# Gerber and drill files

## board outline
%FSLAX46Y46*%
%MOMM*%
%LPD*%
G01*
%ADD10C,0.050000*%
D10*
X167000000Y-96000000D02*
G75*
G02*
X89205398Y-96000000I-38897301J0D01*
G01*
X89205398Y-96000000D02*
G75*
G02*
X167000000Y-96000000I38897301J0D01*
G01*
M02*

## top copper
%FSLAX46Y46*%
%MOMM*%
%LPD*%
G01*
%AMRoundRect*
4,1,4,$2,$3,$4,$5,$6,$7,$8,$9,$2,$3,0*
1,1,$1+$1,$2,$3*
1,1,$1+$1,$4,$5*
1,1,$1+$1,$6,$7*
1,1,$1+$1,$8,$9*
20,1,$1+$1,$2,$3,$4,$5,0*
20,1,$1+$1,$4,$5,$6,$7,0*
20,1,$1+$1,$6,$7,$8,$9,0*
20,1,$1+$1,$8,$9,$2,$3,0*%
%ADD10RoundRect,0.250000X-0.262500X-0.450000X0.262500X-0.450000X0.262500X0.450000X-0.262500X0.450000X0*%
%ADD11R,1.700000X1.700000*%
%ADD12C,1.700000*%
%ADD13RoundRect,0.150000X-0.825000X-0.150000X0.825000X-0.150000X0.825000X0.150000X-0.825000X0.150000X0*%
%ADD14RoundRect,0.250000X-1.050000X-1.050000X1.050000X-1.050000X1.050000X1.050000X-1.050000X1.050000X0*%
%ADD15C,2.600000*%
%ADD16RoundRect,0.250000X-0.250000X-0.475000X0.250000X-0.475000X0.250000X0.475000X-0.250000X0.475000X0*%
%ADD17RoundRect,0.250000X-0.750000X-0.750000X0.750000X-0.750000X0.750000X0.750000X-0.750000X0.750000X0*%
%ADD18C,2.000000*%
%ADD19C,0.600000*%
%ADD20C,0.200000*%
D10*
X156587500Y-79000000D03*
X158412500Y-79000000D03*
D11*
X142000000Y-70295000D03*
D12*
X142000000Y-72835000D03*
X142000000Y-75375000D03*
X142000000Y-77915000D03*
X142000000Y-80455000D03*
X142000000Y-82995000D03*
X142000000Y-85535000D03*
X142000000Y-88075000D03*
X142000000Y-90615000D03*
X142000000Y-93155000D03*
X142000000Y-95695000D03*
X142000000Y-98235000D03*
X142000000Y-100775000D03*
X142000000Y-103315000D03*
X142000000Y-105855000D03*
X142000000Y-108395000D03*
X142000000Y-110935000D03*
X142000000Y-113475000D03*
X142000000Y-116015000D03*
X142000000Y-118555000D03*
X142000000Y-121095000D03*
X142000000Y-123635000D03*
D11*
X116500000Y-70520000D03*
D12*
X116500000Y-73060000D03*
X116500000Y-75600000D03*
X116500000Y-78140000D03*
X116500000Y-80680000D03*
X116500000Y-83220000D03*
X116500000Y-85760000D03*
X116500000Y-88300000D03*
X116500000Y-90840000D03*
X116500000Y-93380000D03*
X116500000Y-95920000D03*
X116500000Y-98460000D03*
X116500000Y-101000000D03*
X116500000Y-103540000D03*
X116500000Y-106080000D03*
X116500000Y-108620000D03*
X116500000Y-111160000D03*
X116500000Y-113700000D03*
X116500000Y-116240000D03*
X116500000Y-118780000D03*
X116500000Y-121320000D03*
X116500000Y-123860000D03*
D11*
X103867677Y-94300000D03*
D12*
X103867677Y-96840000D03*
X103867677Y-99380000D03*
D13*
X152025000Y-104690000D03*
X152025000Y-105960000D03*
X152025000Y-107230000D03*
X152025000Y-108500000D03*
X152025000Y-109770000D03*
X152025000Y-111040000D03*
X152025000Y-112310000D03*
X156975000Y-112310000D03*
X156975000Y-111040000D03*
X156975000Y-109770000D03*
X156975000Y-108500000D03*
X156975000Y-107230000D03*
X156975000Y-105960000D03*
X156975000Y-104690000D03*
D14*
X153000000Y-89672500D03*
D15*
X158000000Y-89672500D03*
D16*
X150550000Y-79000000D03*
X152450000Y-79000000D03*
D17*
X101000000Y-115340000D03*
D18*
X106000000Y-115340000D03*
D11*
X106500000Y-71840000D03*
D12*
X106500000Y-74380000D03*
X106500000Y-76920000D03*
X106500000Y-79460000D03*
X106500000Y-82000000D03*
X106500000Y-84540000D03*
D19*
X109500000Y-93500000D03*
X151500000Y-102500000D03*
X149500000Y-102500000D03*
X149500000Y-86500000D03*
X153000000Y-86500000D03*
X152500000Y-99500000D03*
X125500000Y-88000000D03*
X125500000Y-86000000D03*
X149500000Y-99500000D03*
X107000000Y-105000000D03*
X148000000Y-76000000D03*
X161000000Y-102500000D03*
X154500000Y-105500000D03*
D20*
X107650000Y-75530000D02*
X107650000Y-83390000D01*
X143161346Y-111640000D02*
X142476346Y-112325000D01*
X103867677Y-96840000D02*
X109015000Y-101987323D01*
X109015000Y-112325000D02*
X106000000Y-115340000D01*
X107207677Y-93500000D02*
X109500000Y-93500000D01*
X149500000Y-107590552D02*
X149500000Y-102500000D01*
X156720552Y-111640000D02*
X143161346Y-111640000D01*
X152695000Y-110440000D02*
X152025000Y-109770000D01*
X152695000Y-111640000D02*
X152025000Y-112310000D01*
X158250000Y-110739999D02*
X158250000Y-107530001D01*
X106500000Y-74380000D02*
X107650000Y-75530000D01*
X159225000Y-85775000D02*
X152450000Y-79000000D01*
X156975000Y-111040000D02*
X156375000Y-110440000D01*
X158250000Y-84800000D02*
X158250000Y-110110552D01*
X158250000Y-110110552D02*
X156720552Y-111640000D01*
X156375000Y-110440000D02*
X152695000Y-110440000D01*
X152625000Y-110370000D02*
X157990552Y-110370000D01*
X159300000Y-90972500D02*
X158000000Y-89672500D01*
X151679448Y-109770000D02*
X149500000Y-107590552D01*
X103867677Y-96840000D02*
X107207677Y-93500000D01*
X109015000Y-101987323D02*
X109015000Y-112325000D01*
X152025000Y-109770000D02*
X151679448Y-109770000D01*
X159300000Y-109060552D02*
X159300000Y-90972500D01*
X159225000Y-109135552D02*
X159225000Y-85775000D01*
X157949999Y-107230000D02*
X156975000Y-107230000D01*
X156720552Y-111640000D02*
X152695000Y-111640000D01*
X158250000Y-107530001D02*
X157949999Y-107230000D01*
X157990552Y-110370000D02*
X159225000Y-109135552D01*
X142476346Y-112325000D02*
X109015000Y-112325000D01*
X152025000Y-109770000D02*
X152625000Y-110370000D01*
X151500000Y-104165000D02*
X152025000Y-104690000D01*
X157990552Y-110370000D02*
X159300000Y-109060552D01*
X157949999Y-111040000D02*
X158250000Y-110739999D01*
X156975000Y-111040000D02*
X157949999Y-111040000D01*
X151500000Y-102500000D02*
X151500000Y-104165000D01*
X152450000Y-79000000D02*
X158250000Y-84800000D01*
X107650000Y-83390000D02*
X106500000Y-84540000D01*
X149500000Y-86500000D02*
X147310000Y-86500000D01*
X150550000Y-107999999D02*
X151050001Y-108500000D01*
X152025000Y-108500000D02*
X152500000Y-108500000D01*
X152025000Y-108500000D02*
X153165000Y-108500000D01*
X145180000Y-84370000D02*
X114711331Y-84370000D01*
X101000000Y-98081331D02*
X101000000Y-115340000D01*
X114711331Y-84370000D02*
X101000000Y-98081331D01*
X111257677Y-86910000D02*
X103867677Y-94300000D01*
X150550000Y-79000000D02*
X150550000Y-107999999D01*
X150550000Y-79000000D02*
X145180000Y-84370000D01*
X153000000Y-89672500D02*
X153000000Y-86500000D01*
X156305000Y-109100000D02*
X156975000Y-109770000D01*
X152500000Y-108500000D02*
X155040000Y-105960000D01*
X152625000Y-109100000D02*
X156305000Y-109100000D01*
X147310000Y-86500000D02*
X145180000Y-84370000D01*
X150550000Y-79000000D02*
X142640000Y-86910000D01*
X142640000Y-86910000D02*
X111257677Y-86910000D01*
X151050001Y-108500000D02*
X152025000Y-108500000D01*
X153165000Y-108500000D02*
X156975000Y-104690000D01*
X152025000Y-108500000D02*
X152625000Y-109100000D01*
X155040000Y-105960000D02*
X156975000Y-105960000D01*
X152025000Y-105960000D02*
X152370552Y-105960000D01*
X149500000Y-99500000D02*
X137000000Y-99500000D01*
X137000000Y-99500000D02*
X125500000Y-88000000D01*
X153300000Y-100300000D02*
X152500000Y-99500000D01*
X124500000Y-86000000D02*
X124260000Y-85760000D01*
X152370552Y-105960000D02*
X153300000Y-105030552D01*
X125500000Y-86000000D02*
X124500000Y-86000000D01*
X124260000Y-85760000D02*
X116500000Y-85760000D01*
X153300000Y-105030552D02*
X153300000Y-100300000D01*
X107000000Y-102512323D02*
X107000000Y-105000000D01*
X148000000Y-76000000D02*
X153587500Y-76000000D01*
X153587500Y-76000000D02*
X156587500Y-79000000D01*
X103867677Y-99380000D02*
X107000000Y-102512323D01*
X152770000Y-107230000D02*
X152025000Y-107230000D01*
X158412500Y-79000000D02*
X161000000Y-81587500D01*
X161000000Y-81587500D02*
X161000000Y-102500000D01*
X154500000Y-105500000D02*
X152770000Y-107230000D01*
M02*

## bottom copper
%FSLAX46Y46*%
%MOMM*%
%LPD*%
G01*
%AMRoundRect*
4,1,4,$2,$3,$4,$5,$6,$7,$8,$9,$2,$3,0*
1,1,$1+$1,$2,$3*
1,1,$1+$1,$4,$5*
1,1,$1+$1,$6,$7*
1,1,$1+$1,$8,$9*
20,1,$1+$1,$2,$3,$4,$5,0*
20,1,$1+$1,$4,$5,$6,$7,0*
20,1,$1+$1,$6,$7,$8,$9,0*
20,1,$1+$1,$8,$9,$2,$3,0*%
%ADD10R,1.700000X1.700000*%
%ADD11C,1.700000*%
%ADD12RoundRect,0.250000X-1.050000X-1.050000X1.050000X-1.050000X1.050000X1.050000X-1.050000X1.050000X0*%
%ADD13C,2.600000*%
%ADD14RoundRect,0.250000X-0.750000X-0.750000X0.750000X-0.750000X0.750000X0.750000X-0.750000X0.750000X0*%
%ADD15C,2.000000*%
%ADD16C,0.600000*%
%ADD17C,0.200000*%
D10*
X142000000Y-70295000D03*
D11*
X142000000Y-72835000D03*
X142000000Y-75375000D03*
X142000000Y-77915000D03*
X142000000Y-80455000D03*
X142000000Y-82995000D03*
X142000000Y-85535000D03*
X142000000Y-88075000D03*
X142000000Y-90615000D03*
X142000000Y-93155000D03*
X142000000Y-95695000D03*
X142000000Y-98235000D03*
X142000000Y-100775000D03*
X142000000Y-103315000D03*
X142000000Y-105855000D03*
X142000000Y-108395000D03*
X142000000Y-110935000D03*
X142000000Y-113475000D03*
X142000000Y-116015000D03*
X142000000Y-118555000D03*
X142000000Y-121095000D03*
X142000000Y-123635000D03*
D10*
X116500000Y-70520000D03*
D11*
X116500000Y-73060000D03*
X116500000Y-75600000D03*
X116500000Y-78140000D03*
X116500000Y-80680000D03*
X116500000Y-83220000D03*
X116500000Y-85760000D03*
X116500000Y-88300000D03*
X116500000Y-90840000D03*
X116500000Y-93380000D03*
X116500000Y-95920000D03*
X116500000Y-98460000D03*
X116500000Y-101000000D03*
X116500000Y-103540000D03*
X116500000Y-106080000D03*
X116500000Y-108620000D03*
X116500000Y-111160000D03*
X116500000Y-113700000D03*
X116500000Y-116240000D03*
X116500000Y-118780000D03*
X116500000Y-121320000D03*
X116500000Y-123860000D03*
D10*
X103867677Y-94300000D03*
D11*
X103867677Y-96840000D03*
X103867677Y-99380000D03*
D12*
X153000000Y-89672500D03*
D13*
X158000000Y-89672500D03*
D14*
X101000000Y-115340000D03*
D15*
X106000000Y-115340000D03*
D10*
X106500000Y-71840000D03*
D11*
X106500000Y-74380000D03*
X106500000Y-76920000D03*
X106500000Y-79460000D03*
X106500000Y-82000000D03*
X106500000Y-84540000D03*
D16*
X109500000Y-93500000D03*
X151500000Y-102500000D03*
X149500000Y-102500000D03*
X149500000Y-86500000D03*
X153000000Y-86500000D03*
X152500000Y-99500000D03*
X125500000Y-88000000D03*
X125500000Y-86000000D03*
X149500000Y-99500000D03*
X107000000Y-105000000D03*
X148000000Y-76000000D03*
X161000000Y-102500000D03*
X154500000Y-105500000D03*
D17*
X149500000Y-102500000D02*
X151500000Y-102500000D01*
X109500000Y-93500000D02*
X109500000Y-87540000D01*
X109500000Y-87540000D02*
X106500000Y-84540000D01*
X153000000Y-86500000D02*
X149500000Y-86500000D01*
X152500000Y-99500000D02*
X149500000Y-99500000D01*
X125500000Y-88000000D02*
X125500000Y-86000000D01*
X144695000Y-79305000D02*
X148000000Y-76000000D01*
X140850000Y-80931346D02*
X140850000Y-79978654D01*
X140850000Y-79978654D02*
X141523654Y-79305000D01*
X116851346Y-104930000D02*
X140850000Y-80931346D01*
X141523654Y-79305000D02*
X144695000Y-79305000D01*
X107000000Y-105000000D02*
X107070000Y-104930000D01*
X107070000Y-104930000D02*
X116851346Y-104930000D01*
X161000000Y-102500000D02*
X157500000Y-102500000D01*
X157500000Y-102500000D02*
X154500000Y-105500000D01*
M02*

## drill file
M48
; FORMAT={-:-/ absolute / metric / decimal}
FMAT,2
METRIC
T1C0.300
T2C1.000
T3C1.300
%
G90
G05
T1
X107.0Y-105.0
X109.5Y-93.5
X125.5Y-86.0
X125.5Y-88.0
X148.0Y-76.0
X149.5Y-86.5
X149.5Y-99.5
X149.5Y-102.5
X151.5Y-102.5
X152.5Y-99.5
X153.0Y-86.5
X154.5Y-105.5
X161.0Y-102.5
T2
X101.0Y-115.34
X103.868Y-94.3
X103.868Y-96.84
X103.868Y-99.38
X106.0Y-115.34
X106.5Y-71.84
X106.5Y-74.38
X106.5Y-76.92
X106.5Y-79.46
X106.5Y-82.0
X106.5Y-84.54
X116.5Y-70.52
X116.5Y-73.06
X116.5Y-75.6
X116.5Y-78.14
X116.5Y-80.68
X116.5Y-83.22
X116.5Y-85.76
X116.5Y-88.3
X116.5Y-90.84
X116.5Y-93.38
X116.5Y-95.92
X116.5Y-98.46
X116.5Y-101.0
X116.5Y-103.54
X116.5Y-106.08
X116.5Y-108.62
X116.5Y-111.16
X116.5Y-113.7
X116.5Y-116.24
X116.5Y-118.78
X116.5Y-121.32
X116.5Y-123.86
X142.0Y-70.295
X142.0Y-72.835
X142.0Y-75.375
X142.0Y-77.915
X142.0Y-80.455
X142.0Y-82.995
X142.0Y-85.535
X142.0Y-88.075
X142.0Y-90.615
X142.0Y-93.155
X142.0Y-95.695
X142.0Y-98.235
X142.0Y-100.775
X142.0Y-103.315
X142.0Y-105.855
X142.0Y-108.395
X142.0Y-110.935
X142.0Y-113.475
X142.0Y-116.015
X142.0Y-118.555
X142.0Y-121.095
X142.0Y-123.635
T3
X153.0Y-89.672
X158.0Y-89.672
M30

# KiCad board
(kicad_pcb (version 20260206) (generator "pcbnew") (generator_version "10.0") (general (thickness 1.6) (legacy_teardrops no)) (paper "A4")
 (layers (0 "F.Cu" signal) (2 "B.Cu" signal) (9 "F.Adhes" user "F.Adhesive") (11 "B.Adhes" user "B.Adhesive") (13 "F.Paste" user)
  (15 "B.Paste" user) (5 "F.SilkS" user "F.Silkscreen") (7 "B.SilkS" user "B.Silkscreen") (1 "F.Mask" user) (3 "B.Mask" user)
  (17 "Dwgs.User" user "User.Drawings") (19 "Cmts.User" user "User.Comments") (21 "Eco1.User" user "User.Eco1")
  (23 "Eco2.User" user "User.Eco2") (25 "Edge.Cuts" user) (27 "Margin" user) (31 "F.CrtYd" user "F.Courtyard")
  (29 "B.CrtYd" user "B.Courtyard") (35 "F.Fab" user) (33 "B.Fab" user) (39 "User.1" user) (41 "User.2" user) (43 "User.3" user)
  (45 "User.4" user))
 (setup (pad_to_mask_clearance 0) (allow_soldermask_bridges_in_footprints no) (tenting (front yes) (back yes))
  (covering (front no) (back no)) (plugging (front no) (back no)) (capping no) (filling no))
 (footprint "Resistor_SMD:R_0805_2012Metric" (layer "F.Cu") (at 157.5 79)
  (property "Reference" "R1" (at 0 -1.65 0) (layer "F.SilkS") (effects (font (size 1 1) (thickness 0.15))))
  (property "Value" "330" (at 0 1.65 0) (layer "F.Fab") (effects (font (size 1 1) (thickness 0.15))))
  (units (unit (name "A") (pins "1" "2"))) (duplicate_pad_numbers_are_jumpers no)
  (pad "1" smd roundrect (at -0.9125 0) (size 1.025 1.4) (layers "F.Cu" "F.Mask" "F.Paste") (roundrect_rratio 0.243902)
   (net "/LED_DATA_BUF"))
  (pad "2" smd roundrect (at 0.9125 0) (size 1.025 1.4) (layers "F.Cu" "F.Mask" "F.Paste") (roundrect_rratio 0.243902) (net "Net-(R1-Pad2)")))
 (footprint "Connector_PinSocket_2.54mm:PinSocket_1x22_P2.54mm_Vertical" (layer "F.Cu") (at 142 70.295)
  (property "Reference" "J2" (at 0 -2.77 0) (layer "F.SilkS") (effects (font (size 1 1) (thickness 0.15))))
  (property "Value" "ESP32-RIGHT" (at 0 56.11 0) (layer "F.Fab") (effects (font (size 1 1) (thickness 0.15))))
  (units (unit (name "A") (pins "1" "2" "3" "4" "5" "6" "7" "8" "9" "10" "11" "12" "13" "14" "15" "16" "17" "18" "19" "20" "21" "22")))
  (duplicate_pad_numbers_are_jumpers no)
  (pad "1" thru_hole rect (at 0 0) (size 1.7 1.7) (drill 1) (layers "*.Cu" "*.Mask") (remove_unused_layers no)
   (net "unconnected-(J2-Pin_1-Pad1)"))
  (pad "2" thru_hole circle (at 0 2.54) (size 1.7 1.7) (drill 1) (layers "*.Cu" "*.Mask") (remove_unused_layers no)
   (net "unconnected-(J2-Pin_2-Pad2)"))
  (pad "3" thru_hole circle (at 0 5.08) (size 1.7 1.7) (drill 1) (layers "*.Cu" "*.Mask") (remove_unused_layers no)
   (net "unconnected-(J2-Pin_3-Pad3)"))
  (pad "4" thru_hole circle (at 0 7.62) (size 1.7 1.7) (drill 1) (layers "*.Cu" "*.Mask") (remove_unused_layers no)
   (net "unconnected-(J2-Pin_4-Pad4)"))
  (pad "5" thru_hole circle (at 0 10.16) (size 1.7 1.7) (drill 1) (layers "*.Cu" "*.Mask") (remove_unused_layers no)
   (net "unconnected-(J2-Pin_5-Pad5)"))
  (pad "6" thru_hole circle (at 0 12.7) (size 1.7 1.7) (drill 1) (layers "*.Cu" "*.Mask") (remove_unused_layers no)
   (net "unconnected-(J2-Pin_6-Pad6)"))
  (pad "7" thru_hole circle (at 0 15.24) (size 1.7 1.7) (drill 1) (layers "*.Cu" "*.Mask") (remove_unused_layers no)
   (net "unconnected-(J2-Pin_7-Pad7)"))
  (pad "8" thru_hole circle (at 0 17.78) (size 1.7 1.7) (drill 1) (layers "*.Cu" "*.Mask") (remove_unused_layers no)
   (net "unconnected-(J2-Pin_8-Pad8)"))
  (pad "9" thru_hole circle (at 0 20.32) (size 1.7 1.7) (drill 1) (layers "*.Cu" "*.Mask") (remove_unused_layers no)
   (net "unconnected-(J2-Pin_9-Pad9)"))
  (pad "10" thru_hole circle (at 0 22.86) (size 1.7 1.7) (drill 1) (layers "*.Cu" "*.Mask") (remove_unused_layers no)
   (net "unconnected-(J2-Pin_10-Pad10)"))
  (pad "11" thru_hole circle (at 0 25.4) (size 1.7 1.7) (drill 1) (layers "*.Cu" "*.Mask") (remove_unused_layers no)
   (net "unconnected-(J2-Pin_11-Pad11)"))
  (pad "12" thru_hole circle (at 0 27.94) (size 1.7 1.7) (drill 1) (layers "*.Cu" "*.Mask") (remove_unused_layers no)
   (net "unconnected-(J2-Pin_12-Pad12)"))
  (pad "13" thru_hole circle (at 0 30.48) (size 1.7 1.7) (drill 1) (layers "*.Cu" "*.Mask") (remove_unused_layers no)
   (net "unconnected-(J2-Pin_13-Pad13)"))
  (pad "14" thru_hole circle (at 0 33.02) (size 1.7 1.7) (drill 1) (layers "*.Cu" "*.Mask") (remove_unused_layers no)
   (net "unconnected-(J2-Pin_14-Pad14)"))
  (pad "15" thru_hole circle (at 0 35.56) (size 1.7 1.7) (drill 1) (layers "*.Cu" "*.Mask") (remove_unused_layers no)
   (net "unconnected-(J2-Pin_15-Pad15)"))
  (pad "16" thru_hole circle (at 0 38.1) (size 1.7 1.7) (drill 1) (layers "*.Cu" "*.Mask") (remove_unused_layers no)
   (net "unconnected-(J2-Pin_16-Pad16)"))
  (pad "17" thru_hole circle (at 0 40.64) (size 1.7 1.7) (drill 1) (layers "*.Cu" "*.Mask") (remove_unused_layers no)
   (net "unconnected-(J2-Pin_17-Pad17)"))
  (pad "18" thru_hole circle (at 0 43.18) (size 1.7 1.7) (drill 1) (layers "*.Cu" "*.Mask") (remove_unused_layers no)
   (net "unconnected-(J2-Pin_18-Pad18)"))
  (pad "19" thru_hole circle (at 0 45.72) (size 1.7 1.7) (drill 1) (layers "*.Cu" "*.Mask") (remove_unused_layers no)
   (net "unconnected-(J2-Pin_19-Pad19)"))
  (pad "20" thru_hole circle (at 0 48.26) (size 1.7 1.7) (drill 1) (layers "*.Cu" "*.Mask") (remove_unused_layers no)
   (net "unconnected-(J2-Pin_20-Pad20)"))
  (pad "21" thru_hole circle (at 0 50.8) (size 1.7 1.7) (drill 1) (layers "*.Cu" "*.Mask") (remove_unused_layers no)
   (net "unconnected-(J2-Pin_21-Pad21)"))
  (pad "22" thru_hole circle (at 0 53.34) (size 1.7 1.7) (drill 1) (layers "*.Cu" "*.Mask") (remove_unused_layers no)
   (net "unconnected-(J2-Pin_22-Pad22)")))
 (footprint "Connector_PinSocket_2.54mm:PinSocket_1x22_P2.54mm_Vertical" (layer "F.Cu") (at 116.5 70.52)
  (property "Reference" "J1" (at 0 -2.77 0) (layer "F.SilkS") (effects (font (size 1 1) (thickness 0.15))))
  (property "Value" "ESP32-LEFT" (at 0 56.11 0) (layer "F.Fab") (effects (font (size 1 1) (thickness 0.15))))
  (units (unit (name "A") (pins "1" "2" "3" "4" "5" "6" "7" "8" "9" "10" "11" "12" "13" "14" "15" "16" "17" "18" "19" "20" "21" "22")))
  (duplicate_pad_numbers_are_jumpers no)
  (pad "1" thru_hole rect (at 0 0) (size 1.7 1.7) (drill 1) (layers "*.Cu" "*.Mask") (remove_unused_layers no)
   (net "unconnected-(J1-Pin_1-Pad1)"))
  (pad "2" thru_hole circle (at 0 2.54) (size 1.7 1.7) (drill 1) (layers "*.Cu" "*.Mask") (remove_unused_layers no)
   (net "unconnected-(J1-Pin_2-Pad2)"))
  (pad "3" thru_hole circle (at 0 5.08) (size 1.7 1.7) (drill 1) (layers "*.Cu" "*.Mask") (remove_unused_layers no)
   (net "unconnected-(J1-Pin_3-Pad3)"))
  (pad "4" thru_hole circle (at 0 7.62) (size 1.7 1.7) (drill 1) (layers "*.Cu" "*.Mask") (remove_unused_layers no)
   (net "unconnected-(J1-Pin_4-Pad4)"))
  (pad "5" thru_hole circle (at 0 10.16) (size 1.7 1.7) (drill 1) (layers "*.Cu" "*.Mask") (remove_unused_layers no)
   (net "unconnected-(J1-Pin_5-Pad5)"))
  (pad "6" thru_hole circle (at 0 12.7) (size 1.7 1.7) (drill 1) (layers "*.Cu" "*.Mask") (remove_unused_layers no)
   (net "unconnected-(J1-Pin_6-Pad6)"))
  (pad "7" thru_hole circle (at 0 15.24) (size 1.7 1.7) (drill 1) (layers "*.Cu" "*.Mask") (remove_unused_layers no) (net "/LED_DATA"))
  (pad "8" thru_hole circle (at 0 17.78) (size 1.7 1.7) (drill 1) (layers "*.Cu" "*.Mask") (remove_unused_layers no)
   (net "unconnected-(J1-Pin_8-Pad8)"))
  (pad "9" thru_hole circle (at 0 20.32) (size 1.7 1.7) (drill 1) (layers "*.Cu" "*.Mask") (remove_unused_layers no)
   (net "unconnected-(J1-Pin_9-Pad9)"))
  (pad "10" thru_hole circle (at 0 22.86) (size 1.7 1.7) (drill 1) (layers "*.Cu" "*.Mask") (remove_unused_layers no)
   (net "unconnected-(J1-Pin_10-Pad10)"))
  (pad "11" thru_hole circle (at 0 25.4) (size 1.7 1.7) (drill 1) (layers "*.Cu" "*.Mask") (remove_unused_layers no)
   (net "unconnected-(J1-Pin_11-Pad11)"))
  (pad "12" thru_hole circle (at 0 27.94) (size 1.7 1.7) (drill 1) (layers "*.Cu" "*.Mask") (remove_unused_layers no)
   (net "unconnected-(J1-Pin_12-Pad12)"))
  (pad "13" thru_hole circle (at 0 30.48) (size 1.7 1.7) (drill 1) (layers "*.Cu" "*.Mask") (remove_unused_layers no)
   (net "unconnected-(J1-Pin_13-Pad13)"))
  (pad "14" thru_hole circle (at 0 33.02) (size 1.7 1.7) (drill 1) (layers "*.Cu" "*.Mask") (remove_unused_layers no)
   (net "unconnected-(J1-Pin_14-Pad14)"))
  (pad "15" thru_hole circle (at 0 35.56) (size 1.7 1.7) (drill 1) (layers "*.Cu" "*.Mask") (remove_unused_layers no)
   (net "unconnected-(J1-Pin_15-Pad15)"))
  (pad "16" thru_hole circle (at 0 38.1) (size 1.7 1.7) (drill 1) (layers "*.Cu" "*.Mask") (remove_unused_layers no)
   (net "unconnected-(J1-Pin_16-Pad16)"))
  (pad "17" thru_hole circle (at 0 40.64) (size 1.7 1.7) (drill 1) (layers "*.Cu" "*.Mask") (remove_unused_layers no)
   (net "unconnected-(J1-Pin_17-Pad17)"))
  (pad "18" thru_hole circle (at 0 43.18) (size 1.7 1.7) (drill 1) (layers "*.Cu" "*.Mask") (remove_unused_layers no)
   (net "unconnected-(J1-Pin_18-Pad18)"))
  (pad "19" thru_hole circle (at 0 45.72) (size 1.7 1.7) (drill 1) (layers "*.Cu" "*.Mask") (remove_unused_layers no)
   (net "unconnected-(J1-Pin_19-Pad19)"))
  (pad "20" thru_hole circle (at 0 48.26) (size 1.7 1.7) (drill 1) (layers "*.Cu" "*.Mask") (remove_unused_layers no)
   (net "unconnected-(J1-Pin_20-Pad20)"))
  (pad "21" thru_hole circle (at 0 50.8) (size 1.7 1.7) (drill 1) (layers "*.Cu" "*.Mask") (remove_unused_layers no)
   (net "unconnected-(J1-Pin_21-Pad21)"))
  (pad "22" thru_hole circle (at 0 53.34) (size 1.7 1.7) (drill 1) (layers "*.Cu" "*.Mask") (remove_unused_layers no)
   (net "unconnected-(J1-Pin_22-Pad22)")))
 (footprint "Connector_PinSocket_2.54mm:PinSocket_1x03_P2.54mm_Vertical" (layer "F.Cu") (at 103.867677 94.3)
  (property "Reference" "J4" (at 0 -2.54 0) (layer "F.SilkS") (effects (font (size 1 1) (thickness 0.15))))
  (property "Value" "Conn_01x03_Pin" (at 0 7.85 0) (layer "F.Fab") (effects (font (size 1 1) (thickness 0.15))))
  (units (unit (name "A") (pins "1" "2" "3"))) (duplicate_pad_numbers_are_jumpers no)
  (pad "1" thru_hole rect (at 0 0) (size 1.7 1.7) (drill 1) (layers "*.Cu" "*.Mask") (remove_unused_layers no) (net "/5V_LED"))
  (pad "2" thru_hole circle (at 0 2.54) (size 1.7 1.7) (drill 1) (layers "*.Cu" "*.Mask") (remove_unused_layers no) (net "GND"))
  (pad "3" thru_hole circle (at 0 5.08) (size 1.7 1.7) (drill 1) (layers "*.Cu" "*.Mask") (remove_unused_layers no) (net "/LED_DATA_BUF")))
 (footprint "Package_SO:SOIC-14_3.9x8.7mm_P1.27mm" (layer "F.Cu") (at 154.5 108.5)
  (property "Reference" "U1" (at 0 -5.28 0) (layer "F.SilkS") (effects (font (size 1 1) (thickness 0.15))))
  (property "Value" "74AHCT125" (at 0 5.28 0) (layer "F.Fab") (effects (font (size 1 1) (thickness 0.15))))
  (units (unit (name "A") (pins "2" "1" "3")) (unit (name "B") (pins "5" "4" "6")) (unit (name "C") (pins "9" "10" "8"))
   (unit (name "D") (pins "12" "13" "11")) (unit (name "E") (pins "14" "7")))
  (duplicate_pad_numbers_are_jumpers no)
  (pad "1" smd roundrect (at -2.475 -3.81) (size 1.95 0.6) (layers "F.Cu" "F.Mask" "F.Paste") (roundrect_rratio 0.25) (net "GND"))
  (pad "2" smd roundrect (at -2.475 -2.54) (size 1.95 0.6) (layers "F.Cu" "F.Mask" "F.Paste") (roundrect_rratio 0.25) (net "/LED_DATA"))
  (pad "3" smd roundrect (at -2.475 -1.27) (size 1.95 0.6) (layers "F.Cu" "F.Mask" "F.Paste") (roundrect_rratio 0.25) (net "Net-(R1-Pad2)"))
  (pad "4" smd roundrect (at -2.475 0) (size 1.95 0.6) (layers "F.Cu" "F.Mask" "F.Paste") (roundrect_rratio 0.25) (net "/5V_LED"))
  (pad "5" smd roundrect (at -2.475 1.27) (size 1.95 0.6) (layers "F.Cu" "F.Mask" "F.Paste") (roundrect_rratio 0.25) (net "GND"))
  (pad "6" smd roundrect (at -2.475 2.54) (size 1.95 0.6) (layers "F.Cu" "F.Mask" "F.Paste") (roundrect_rratio 0.25)
   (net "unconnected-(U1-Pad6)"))
  (pad "7" smd roundrect (at -2.475 3.81) (size 1.95 0.6) (layers "F.Cu" "F.Mask" "F.Paste") (roundrect_rratio 0.25) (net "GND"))
  (pad "8" smd roundrect (at 2.475 3.81) (size 1.95 0.6) (layers "F.Cu" "F.Mask" "F.Paste") (roundrect_rratio 0.25)
   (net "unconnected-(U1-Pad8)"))
  (pad "9" smd roundrect (at 2.475 2.54) (size 1.95 0.6) (layers "F.Cu" "F.Mask" "F.Paste") (roundrect_rratio 0.25) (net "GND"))
  (pad "10" smd roundrect (at 2.475 1.27) (size 1.95 0.6) (layers "F.Cu" "F.Mask" "F.Paste") (roundrect_rratio 0.25) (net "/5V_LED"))
  (pad "11" smd roundrect (at 2.475 0) (size 1.95 0.6) (layers "F.Cu" "F.Mask" "F.Paste") (roundrect_rratio 0.25)
   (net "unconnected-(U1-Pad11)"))
  (pad "12" smd roundrect (at 2.475 -1.27) (size 1.95 0.6) (layers "F.Cu" "F.Mask" "F.Paste") (roundrect_rratio 0.25) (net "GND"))
  (pad "13" smd roundrect (at 2.475 -2.54) (size 1.95 0.6) (layers "F.Cu" "F.Mask" "F.Paste") (roundrect_rratio 0.25) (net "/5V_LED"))
  (pad "14" smd roundrect (at 2.475 -3.81) (size 1.95 0.6) (layers "F.Cu" "F.Mask" "F.Paste") (roundrect_rratio 0.25) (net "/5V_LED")))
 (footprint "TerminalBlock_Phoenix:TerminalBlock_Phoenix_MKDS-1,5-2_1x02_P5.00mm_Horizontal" (layer "F.Cu") (at 153 89.6725)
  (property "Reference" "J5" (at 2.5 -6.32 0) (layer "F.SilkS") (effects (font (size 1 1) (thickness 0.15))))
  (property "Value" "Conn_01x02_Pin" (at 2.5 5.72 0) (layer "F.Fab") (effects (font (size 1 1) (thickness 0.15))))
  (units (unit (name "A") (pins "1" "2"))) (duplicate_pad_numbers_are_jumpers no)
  (pad "1" thru_hole roundrect (at 0 0) (size 2.6 2.6) (drill 1.3) (layers "*.Cu" "*.Mask") (remove_unused_layers no)
   (roundrect_rratio 0.096154) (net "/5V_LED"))
  (pad "2" thru_hole circle (at 5 0) (size 2.6 2.6) (drill 1.3) (layers "*.Cu" "*.Mask") (remove_unused_layers no) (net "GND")))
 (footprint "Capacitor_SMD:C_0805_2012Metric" (layer "F.Cu") (at 151.5 79)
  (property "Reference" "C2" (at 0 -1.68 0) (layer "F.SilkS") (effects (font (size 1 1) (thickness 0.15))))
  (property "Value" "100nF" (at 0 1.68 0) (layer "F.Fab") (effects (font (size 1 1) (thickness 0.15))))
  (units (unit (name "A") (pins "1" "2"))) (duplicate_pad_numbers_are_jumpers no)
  (pad "1" smd roundrect (at -0.95 0) (size 1 1.45) (layers "F.Cu" "F.Mask" "F.Paste") (roundrect_rratio 0.25) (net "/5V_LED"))
  (pad "2" smd roundrect (at 0.95 0) (size 1 1.45) (layers "F.Cu" "F.Mask" "F.Paste") (roundrect_rratio 0.25) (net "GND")))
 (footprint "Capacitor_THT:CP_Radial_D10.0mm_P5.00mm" (layer "F.Cu") (at 101 115.34)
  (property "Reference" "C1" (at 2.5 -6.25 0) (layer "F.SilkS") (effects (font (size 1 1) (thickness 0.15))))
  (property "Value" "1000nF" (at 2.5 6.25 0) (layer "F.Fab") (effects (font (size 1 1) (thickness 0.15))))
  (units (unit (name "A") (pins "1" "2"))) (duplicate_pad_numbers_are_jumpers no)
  (pad "1" thru_hole roundrect (at 0 0) (size 2 2) (drill 1) (layers "*.Cu" "*.Mask") (remove_unused_layers no) (roundrect_rratio 0.125)
   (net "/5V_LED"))
  (pad "2" thru_hole circle (at 5 0) (size 2 2) (drill 1) (layers "*.Cu" "*.Mask") (remove_unused_layers no) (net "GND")))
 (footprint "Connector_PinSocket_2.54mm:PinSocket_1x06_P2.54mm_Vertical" (layer "F.Cu") (at 106.5 71.84)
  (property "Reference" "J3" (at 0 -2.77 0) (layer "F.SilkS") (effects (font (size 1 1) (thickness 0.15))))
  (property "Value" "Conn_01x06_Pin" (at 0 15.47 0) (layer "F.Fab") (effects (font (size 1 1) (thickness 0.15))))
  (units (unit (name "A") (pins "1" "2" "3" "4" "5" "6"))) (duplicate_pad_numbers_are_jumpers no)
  (pad "1" thru_hole rect (at 0 0) (size 1.7 1.7) (drill 1) (layers "*.Cu" "*.Mask") (remove_unused_layers no) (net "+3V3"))
  (pad "2" thru_hole circle (at 0 2.54) (size 1.7 1.7) (drill 1) (layers "*.Cu" "*.Mask") (remove_unused_layers no) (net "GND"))
  (pad "3" thru_hole circle (at 0 5.08) (size 1.7 1.7) (drill 1) (layers "*.Cu" "*.Mask") (remove_unused_layers no) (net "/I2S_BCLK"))
  (pad "4" thru_hole circle (at 0 7.62) (size 1.7 1.7) (drill 1) (layers "*.Cu" "*.Mask") (remove_unused_layers no) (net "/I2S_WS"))
  (pad "5" thru_hole circle (at 0 10.16) (size 1.7 1.7) (drill 1) (layers "*.Cu" "*.Mask") (remove_unused_layers no) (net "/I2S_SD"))
  (pad "6" thru_hole circle (at 0 12.7) (size 1.7 1.7) (drill 1) (layers "*.Cu" "*.Mask") (remove_unused_layers no) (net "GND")))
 (gr_circle (center 128.102699 96) (end 155.102699 124) (stroke (width 0.05) (type default)) (fill no) (layer "Edge.Cuts"))
 (segment (start 107.65 75.53) (end 107.65 83.39) (width 0.2) (layer "F.Cu") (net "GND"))
 (segment (start 143.161346 111.64) (end 142.476346 112.325) (width 0.2) (layer "F.Cu") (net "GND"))
 (segment (start 103.867677 96.84) (end 109.015 101.987323) (width 0.2) (layer "F.Cu") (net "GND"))
 (segment (start 109.015 112.325) (end 106 115.34) (width 0.2) (layer "F.Cu") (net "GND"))
 (segment (start 107.207677 93.5) (end 109.5 93.5) (width 0.2) (layer "F.Cu") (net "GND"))
 (segment (start 149.5 107.590552) (end 149.5 102.5) (width 0.2) (layer "F.Cu") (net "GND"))
 (segment (start 156.720552 111.64) (end 143.161346 111.64) (width 0.2) (layer "F.Cu") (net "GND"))
 (segment (start 152.695 110.44) (end 152.025 109.77) (width 0.2) (layer "F.Cu") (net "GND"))
 (segment (start 152.695 111.64) (end 152.025 112.31) (width 0.2) (layer "F.Cu") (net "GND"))
 (segment (start 158.25 110.739999) (end 158.25 107.530001) (width 0.2) (layer "F.Cu") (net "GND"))
 (segment (start 106.5 74.38) (end 107.65 75.53) (width 0.2) (layer "F.Cu") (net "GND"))
 (segment (start 159.225 85.775) (end 152.45 79) (width 0.2) (layer "F.Cu") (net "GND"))
 (segment (start 156.975 111.04) (end 156.375 110.44) (width 0.2) (layer "F.Cu") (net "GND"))
 (segment (start 158.25 84.8) (end 158.25 110.110552) (width 0.2) (layer "F.Cu") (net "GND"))
 (segment (start 158.25 110.110552) (end 156.720552 111.64) (width 0.2) (layer "F.Cu") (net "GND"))
 (segment (start 156.375 110.44) (end 152.695 110.44) (width 0.2) (layer "F.Cu") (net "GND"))
 (segment (start 152.625 110.37) (end 157.990552 110.37) (width 0.2) (layer "F.Cu") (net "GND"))
 (segment (start 159.3 90.9725) (end 158 89.6725) (width 0.2) (layer "F.Cu") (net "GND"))
 (segment (start 151.679448 109.77) (end 149.5 107.590552) (width 0.2) (layer "F.Cu") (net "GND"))
 (segment (start 103.867677 96.84) (end 107.207677 93.5) (width 0.2) (layer "F.Cu") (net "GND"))
 (segment (start 109.015 101.987323) (end 109.015 112.325) (width 0.2) (layer "F.Cu") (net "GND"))
 (segment (start 152.025 109.77) (end 151.679448 109.77) (width 0.2) (layer "F.Cu") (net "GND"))
 (segment (start 159.3 109.060552) (end 159.3 90.9725) (width 0.2) (layer "F.Cu") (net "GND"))
 (segment (start 159.225 109.135552) (end 159.225 85.775) (width 0.2) (layer "F.Cu") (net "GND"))
 (segment (start 157.949999 107.23) (end 156.975 107.23) (width 0.2) (layer "F.Cu") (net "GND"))
 (segment (start 156.720552 111.64) (end 152.695 111.64) (width 0.2) (layer "F.Cu") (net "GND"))
 (segment (start 158.25 107.530001) (end 157.949999 107.23) (width 0.2) (layer "F.Cu") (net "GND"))
 (segment (start 157.990552 110.37) (end 159.225 109.135552) (width 0.2) (layer "F.Cu") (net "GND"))
 (segment (start 142.476346 112.325) (end 109.015 112.325) (width 0.2) (layer "F.Cu") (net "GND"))
 (segment (start 152.025 109.77) (end 152.625 110.37) (width 0.2) (layer "F.Cu") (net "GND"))
 (segment (start 151.5 104.165) (end 152.025 104.69) (width 0.2) (layer "F.Cu") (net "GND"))
 (segment (start 157.990552 110.37) (end 159.3 109.060552) (width 0.2) (layer "F.Cu") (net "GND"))
 (segment (start 157.949999 111.04) (end 158.25 110.739999) (width 0.2) (layer "F.Cu") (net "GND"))
 (segment (start 156.975 111.04) (end 157.949999 111.04) (width 0.2) (layer "F.Cu") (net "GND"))
 (segment (start 151.5 102.5) (end 151.5 104.165) (width 0.2) (layer "F.Cu") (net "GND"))
 (segment (start 152.45 79) (end 158.25 84.8) (width 0.2) (layer "F.Cu") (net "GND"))
 (segment (start 107.65 83.39) (end 106.5 84.54) (width 0.2) (layer "F.Cu") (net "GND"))
 (via (at 109.5 93.5) (size 0.6) (drill 0.3) (layers "F.Cu" "B.Cu") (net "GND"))
 (via (at 151.5 102.5) (size 0.6) (drill 0.3) (layers "F.Cu" "B.Cu") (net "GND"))
 (via (at 149.5 102.5) (size 0.6) (drill 0.3) (layers "F.Cu" "B.Cu") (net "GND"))
 (segment (start 149.5 102.5) (end 151.5 102.5) (width 0.2) (layer "B.Cu") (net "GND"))
 (segment (start 109.5 93.5) (end 109.5 87.54) (width 0.2) (layer "B.Cu") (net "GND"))
 (segment (start 109.5 87.54) (end 106.5 84.54) (width 0.2) (layer "B.Cu") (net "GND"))
 (segment (start 149.5 86.5) (end 147.31 86.5) (width 0.2) (layer "F.Cu") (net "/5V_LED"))
 (segment (start 150.55 107.999999) (end 151.050001 108.5) (width 0.2) (layer "F.Cu") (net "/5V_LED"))
 (segment (start 152.025 108.5) (end 152.5 108.5) (width 0.2) (layer "F.Cu") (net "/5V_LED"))
 (segment (start 152.025 108.5) (end 153.165 108.5) (width 0.2) (layer "F.Cu") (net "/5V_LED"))
 (segment (start 145.18 84.37) (end 114.711331 84.37) (width 0.2) (layer "F.Cu") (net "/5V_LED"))
 (segment (start 101 98.081331) (end 101 115.34) (width 0.2) (layer "F.Cu") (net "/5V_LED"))
 (segment (start 114.711331 84.37) (end 101 98.081331) (width 0.2) (layer "F.Cu") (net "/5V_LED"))
 (segment (start 111.257677 86.91) (end 103.867677 94.3) (width 0.2) (layer "F.Cu") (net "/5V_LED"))
 (segment (start 150.55 79) (end 150.55 107.999999) (width 0.2) (layer "F.Cu") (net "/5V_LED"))
 (segment (start 150.55 79) (end 145.18 84.37) (width 0.2) (layer "F.Cu") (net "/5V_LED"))
 (segment (start 153 89.6725) (end 153 86.5) (width 0.2) (layer "F.Cu") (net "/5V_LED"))
 (segment (start 156.305 109.1) (end 156.975 109.77) (width 0.2) (layer "F.Cu") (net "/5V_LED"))
 (segment (start 152.5 108.5) (end 155.04 105.96) (width 0.2) (layer "F.Cu") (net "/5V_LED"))
 (segment (start 152.625 109.1) (end 156.305 109.1) (width 0.2) (layer "F.Cu") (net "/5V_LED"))
 (segment (start 147.31 86.5) (end 145.18 84.37) (width 0.2) (layer "F.Cu") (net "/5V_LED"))
 (segment (start 150.55 79) (end 142.64 86.91) (width 0.2) (layer "F.Cu") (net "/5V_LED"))
 (segment (start 142.64 86.91) (end 111.257677 86.91) (width 0.2) (layer "F.Cu") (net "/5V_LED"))
 (segment (start 151.050001 108.5) (end 152.025 108.5) (width 0.2) (layer "F.Cu") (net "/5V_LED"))
 (segment (start 153.165 108.5) (end 156.975 104.69) (width 0.2) (layer "F.Cu") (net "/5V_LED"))
 (segment (start 152.025 108.5) (end 152.625 109.1) (width 0.2) (layer "F.Cu") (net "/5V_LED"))
 (segment (start 155.04 105.96) (end 156.975 105.96) (width 0.2) (layer "F.Cu") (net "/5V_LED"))
 (via (at 149.5 86.5) (size 0.6) (drill 0.3) (layers "F.Cu" "B.Cu") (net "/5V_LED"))
 (via (at 153 86.5) (size 0.6) (drill 0.3) (layers "F.Cu" "B.Cu") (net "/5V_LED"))
 (segment (start 153 86.5) (end 149.5 86.5) (width 0.2) (layer "B.Cu") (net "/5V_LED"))
 (segment (start 152.025 105.96) (end 152.370552 105.96) (width 0.2) (layer "F.Cu") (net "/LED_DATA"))
 (segment (start 149.5 99.5) (end 137 99.5) (width 0.2) (layer "F.Cu") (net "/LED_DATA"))
 (segment (start 137 99.5) (end 125.5 88) (width 0.2) (layer "F.Cu") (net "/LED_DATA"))
 (segment (start 153.3 100.3) (end 152.5 99.5) (width 0.2) (layer "F.Cu") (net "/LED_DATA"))
 (segment (start 124.5 86) (end 124.26 85.76) (width 0.2) (layer "F.Cu") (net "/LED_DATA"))
 (segment (start 152.370552 105.96) (end 153.3 105.030552) (width 0.2) (layer "F.Cu") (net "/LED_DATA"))
 (segment (start 125.5 86) (end 124.5 86) (width 0.2) (layer "F.Cu") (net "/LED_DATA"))
 (segment (start 124.26 85.76) (end 116.5 85.76) (width 0.2) (layer "F.Cu") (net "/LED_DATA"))
 (segment (start 153.3 105.030552) (end 153.3 100.3) (width 0.2) (layer "F.Cu") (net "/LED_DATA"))
 (via (at 152.5 99.5) (size 0.6) (drill 0.3) (layers "F.Cu" "B.Cu") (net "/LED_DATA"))
 (via (at 125.5 88) (size 0.6) (drill 0.3) (layers "F.Cu" "B.Cu") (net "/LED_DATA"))
 (via (at 125.5 86) (size 0.6) (drill 0.3) (layers "F.Cu" "B.Cu") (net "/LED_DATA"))
 (via (at 149.5 99.5) (size 0.6) (drill 0.3) (layers "F.Cu" "B.Cu") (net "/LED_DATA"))
 (segment (start 152.5 99.5) (end 149.5 99.5) (width 0.2) (layer "B.Cu") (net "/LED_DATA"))
 (segment (start 125.5 88) (end 125.5 86) (width 0.2) (layer "B.Cu") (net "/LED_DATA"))
 (segment (start 107 102.512323) (end 107 105) (width 0.2) (layer "F.Cu") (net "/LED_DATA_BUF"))
 (segment (start 148 76) (end 153.5875 76) (width 0.2) (layer "F.Cu") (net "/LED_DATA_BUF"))
 (segment (start 153.5875 76) (end 156.5875 79) (width 0.2) (layer "F.Cu") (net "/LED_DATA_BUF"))
 (segment (start 103.867677 99.38) (end 107 102.512323) (width 0.2) (layer "F.Cu") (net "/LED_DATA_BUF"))
 (via (at 107 105) (size 0.6) (drill 0.3) (layers "F.Cu" "B.Cu") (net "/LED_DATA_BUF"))
 (via (at 148 76) (size 0.6) (drill 0.3) (layers "F.Cu" "B.Cu") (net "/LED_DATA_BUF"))
 (segment (start 144.695 79.305) (end 148 76) (width 0.2) (layer "B.Cu") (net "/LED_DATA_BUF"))
 (segment (start 140.85 80.931346) (end 140.85 79.978654) (width 0.2) (layer "B.Cu") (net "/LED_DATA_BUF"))
 (segment (start 140.85 79.978654) (end 141.523654 79.305) (width 0.2) (layer "B.Cu") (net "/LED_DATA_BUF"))
 (segment (start 116.851346 104.93) (end 140.85 80.931346) (width 0.2) (layer "B.Cu") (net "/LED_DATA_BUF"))
 (segment (start 141.523654 79.305) (end 144.695 79.305) (width 0.2) (layer "B.Cu") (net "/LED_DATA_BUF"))
 (segment (start 107 105) (end 107.07 104.93) (width 0.2) (layer "B.Cu") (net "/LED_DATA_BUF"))
 (segment (start 107.07 104.93) (end 116.851346 104.93) (width 0.2) (layer "B.Cu") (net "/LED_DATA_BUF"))
 (segment (start 152.77 107.23) (end 152.025 107.23) (width 0.2) (layer "F.Cu") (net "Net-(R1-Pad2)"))
 (segment (start 158.4125 79) (end 161 81.5875) (width 0.2) (layer "F.Cu") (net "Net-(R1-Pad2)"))
 (segment (start 161 81.5875) (end 161 102.5) (width 0.2) (layer "F.Cu") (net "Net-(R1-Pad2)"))
 (segment (start 154.5 105.5) (end 152.77 107.23) (width 0.2) (layer "F.Cu") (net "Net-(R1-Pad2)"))
 (via (at 161 102.5) (size 0.6) (drill 0.3) (layers "F.Cu" "B.Cu") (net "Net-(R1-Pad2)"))
 (via (at 154.5 105.5) (size 0.6) (drill 0.3) (layers "F.Cu" "B.Cu") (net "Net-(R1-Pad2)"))
 (segment (start 161 102.5) (end 157.5 102.5) (width 0.2) (layer "B.Cu") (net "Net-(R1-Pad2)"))
 (segment (start 157.5 102.5) (end 154.5 105.5) (width 0.2) (layer "B.Cu") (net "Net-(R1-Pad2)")))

